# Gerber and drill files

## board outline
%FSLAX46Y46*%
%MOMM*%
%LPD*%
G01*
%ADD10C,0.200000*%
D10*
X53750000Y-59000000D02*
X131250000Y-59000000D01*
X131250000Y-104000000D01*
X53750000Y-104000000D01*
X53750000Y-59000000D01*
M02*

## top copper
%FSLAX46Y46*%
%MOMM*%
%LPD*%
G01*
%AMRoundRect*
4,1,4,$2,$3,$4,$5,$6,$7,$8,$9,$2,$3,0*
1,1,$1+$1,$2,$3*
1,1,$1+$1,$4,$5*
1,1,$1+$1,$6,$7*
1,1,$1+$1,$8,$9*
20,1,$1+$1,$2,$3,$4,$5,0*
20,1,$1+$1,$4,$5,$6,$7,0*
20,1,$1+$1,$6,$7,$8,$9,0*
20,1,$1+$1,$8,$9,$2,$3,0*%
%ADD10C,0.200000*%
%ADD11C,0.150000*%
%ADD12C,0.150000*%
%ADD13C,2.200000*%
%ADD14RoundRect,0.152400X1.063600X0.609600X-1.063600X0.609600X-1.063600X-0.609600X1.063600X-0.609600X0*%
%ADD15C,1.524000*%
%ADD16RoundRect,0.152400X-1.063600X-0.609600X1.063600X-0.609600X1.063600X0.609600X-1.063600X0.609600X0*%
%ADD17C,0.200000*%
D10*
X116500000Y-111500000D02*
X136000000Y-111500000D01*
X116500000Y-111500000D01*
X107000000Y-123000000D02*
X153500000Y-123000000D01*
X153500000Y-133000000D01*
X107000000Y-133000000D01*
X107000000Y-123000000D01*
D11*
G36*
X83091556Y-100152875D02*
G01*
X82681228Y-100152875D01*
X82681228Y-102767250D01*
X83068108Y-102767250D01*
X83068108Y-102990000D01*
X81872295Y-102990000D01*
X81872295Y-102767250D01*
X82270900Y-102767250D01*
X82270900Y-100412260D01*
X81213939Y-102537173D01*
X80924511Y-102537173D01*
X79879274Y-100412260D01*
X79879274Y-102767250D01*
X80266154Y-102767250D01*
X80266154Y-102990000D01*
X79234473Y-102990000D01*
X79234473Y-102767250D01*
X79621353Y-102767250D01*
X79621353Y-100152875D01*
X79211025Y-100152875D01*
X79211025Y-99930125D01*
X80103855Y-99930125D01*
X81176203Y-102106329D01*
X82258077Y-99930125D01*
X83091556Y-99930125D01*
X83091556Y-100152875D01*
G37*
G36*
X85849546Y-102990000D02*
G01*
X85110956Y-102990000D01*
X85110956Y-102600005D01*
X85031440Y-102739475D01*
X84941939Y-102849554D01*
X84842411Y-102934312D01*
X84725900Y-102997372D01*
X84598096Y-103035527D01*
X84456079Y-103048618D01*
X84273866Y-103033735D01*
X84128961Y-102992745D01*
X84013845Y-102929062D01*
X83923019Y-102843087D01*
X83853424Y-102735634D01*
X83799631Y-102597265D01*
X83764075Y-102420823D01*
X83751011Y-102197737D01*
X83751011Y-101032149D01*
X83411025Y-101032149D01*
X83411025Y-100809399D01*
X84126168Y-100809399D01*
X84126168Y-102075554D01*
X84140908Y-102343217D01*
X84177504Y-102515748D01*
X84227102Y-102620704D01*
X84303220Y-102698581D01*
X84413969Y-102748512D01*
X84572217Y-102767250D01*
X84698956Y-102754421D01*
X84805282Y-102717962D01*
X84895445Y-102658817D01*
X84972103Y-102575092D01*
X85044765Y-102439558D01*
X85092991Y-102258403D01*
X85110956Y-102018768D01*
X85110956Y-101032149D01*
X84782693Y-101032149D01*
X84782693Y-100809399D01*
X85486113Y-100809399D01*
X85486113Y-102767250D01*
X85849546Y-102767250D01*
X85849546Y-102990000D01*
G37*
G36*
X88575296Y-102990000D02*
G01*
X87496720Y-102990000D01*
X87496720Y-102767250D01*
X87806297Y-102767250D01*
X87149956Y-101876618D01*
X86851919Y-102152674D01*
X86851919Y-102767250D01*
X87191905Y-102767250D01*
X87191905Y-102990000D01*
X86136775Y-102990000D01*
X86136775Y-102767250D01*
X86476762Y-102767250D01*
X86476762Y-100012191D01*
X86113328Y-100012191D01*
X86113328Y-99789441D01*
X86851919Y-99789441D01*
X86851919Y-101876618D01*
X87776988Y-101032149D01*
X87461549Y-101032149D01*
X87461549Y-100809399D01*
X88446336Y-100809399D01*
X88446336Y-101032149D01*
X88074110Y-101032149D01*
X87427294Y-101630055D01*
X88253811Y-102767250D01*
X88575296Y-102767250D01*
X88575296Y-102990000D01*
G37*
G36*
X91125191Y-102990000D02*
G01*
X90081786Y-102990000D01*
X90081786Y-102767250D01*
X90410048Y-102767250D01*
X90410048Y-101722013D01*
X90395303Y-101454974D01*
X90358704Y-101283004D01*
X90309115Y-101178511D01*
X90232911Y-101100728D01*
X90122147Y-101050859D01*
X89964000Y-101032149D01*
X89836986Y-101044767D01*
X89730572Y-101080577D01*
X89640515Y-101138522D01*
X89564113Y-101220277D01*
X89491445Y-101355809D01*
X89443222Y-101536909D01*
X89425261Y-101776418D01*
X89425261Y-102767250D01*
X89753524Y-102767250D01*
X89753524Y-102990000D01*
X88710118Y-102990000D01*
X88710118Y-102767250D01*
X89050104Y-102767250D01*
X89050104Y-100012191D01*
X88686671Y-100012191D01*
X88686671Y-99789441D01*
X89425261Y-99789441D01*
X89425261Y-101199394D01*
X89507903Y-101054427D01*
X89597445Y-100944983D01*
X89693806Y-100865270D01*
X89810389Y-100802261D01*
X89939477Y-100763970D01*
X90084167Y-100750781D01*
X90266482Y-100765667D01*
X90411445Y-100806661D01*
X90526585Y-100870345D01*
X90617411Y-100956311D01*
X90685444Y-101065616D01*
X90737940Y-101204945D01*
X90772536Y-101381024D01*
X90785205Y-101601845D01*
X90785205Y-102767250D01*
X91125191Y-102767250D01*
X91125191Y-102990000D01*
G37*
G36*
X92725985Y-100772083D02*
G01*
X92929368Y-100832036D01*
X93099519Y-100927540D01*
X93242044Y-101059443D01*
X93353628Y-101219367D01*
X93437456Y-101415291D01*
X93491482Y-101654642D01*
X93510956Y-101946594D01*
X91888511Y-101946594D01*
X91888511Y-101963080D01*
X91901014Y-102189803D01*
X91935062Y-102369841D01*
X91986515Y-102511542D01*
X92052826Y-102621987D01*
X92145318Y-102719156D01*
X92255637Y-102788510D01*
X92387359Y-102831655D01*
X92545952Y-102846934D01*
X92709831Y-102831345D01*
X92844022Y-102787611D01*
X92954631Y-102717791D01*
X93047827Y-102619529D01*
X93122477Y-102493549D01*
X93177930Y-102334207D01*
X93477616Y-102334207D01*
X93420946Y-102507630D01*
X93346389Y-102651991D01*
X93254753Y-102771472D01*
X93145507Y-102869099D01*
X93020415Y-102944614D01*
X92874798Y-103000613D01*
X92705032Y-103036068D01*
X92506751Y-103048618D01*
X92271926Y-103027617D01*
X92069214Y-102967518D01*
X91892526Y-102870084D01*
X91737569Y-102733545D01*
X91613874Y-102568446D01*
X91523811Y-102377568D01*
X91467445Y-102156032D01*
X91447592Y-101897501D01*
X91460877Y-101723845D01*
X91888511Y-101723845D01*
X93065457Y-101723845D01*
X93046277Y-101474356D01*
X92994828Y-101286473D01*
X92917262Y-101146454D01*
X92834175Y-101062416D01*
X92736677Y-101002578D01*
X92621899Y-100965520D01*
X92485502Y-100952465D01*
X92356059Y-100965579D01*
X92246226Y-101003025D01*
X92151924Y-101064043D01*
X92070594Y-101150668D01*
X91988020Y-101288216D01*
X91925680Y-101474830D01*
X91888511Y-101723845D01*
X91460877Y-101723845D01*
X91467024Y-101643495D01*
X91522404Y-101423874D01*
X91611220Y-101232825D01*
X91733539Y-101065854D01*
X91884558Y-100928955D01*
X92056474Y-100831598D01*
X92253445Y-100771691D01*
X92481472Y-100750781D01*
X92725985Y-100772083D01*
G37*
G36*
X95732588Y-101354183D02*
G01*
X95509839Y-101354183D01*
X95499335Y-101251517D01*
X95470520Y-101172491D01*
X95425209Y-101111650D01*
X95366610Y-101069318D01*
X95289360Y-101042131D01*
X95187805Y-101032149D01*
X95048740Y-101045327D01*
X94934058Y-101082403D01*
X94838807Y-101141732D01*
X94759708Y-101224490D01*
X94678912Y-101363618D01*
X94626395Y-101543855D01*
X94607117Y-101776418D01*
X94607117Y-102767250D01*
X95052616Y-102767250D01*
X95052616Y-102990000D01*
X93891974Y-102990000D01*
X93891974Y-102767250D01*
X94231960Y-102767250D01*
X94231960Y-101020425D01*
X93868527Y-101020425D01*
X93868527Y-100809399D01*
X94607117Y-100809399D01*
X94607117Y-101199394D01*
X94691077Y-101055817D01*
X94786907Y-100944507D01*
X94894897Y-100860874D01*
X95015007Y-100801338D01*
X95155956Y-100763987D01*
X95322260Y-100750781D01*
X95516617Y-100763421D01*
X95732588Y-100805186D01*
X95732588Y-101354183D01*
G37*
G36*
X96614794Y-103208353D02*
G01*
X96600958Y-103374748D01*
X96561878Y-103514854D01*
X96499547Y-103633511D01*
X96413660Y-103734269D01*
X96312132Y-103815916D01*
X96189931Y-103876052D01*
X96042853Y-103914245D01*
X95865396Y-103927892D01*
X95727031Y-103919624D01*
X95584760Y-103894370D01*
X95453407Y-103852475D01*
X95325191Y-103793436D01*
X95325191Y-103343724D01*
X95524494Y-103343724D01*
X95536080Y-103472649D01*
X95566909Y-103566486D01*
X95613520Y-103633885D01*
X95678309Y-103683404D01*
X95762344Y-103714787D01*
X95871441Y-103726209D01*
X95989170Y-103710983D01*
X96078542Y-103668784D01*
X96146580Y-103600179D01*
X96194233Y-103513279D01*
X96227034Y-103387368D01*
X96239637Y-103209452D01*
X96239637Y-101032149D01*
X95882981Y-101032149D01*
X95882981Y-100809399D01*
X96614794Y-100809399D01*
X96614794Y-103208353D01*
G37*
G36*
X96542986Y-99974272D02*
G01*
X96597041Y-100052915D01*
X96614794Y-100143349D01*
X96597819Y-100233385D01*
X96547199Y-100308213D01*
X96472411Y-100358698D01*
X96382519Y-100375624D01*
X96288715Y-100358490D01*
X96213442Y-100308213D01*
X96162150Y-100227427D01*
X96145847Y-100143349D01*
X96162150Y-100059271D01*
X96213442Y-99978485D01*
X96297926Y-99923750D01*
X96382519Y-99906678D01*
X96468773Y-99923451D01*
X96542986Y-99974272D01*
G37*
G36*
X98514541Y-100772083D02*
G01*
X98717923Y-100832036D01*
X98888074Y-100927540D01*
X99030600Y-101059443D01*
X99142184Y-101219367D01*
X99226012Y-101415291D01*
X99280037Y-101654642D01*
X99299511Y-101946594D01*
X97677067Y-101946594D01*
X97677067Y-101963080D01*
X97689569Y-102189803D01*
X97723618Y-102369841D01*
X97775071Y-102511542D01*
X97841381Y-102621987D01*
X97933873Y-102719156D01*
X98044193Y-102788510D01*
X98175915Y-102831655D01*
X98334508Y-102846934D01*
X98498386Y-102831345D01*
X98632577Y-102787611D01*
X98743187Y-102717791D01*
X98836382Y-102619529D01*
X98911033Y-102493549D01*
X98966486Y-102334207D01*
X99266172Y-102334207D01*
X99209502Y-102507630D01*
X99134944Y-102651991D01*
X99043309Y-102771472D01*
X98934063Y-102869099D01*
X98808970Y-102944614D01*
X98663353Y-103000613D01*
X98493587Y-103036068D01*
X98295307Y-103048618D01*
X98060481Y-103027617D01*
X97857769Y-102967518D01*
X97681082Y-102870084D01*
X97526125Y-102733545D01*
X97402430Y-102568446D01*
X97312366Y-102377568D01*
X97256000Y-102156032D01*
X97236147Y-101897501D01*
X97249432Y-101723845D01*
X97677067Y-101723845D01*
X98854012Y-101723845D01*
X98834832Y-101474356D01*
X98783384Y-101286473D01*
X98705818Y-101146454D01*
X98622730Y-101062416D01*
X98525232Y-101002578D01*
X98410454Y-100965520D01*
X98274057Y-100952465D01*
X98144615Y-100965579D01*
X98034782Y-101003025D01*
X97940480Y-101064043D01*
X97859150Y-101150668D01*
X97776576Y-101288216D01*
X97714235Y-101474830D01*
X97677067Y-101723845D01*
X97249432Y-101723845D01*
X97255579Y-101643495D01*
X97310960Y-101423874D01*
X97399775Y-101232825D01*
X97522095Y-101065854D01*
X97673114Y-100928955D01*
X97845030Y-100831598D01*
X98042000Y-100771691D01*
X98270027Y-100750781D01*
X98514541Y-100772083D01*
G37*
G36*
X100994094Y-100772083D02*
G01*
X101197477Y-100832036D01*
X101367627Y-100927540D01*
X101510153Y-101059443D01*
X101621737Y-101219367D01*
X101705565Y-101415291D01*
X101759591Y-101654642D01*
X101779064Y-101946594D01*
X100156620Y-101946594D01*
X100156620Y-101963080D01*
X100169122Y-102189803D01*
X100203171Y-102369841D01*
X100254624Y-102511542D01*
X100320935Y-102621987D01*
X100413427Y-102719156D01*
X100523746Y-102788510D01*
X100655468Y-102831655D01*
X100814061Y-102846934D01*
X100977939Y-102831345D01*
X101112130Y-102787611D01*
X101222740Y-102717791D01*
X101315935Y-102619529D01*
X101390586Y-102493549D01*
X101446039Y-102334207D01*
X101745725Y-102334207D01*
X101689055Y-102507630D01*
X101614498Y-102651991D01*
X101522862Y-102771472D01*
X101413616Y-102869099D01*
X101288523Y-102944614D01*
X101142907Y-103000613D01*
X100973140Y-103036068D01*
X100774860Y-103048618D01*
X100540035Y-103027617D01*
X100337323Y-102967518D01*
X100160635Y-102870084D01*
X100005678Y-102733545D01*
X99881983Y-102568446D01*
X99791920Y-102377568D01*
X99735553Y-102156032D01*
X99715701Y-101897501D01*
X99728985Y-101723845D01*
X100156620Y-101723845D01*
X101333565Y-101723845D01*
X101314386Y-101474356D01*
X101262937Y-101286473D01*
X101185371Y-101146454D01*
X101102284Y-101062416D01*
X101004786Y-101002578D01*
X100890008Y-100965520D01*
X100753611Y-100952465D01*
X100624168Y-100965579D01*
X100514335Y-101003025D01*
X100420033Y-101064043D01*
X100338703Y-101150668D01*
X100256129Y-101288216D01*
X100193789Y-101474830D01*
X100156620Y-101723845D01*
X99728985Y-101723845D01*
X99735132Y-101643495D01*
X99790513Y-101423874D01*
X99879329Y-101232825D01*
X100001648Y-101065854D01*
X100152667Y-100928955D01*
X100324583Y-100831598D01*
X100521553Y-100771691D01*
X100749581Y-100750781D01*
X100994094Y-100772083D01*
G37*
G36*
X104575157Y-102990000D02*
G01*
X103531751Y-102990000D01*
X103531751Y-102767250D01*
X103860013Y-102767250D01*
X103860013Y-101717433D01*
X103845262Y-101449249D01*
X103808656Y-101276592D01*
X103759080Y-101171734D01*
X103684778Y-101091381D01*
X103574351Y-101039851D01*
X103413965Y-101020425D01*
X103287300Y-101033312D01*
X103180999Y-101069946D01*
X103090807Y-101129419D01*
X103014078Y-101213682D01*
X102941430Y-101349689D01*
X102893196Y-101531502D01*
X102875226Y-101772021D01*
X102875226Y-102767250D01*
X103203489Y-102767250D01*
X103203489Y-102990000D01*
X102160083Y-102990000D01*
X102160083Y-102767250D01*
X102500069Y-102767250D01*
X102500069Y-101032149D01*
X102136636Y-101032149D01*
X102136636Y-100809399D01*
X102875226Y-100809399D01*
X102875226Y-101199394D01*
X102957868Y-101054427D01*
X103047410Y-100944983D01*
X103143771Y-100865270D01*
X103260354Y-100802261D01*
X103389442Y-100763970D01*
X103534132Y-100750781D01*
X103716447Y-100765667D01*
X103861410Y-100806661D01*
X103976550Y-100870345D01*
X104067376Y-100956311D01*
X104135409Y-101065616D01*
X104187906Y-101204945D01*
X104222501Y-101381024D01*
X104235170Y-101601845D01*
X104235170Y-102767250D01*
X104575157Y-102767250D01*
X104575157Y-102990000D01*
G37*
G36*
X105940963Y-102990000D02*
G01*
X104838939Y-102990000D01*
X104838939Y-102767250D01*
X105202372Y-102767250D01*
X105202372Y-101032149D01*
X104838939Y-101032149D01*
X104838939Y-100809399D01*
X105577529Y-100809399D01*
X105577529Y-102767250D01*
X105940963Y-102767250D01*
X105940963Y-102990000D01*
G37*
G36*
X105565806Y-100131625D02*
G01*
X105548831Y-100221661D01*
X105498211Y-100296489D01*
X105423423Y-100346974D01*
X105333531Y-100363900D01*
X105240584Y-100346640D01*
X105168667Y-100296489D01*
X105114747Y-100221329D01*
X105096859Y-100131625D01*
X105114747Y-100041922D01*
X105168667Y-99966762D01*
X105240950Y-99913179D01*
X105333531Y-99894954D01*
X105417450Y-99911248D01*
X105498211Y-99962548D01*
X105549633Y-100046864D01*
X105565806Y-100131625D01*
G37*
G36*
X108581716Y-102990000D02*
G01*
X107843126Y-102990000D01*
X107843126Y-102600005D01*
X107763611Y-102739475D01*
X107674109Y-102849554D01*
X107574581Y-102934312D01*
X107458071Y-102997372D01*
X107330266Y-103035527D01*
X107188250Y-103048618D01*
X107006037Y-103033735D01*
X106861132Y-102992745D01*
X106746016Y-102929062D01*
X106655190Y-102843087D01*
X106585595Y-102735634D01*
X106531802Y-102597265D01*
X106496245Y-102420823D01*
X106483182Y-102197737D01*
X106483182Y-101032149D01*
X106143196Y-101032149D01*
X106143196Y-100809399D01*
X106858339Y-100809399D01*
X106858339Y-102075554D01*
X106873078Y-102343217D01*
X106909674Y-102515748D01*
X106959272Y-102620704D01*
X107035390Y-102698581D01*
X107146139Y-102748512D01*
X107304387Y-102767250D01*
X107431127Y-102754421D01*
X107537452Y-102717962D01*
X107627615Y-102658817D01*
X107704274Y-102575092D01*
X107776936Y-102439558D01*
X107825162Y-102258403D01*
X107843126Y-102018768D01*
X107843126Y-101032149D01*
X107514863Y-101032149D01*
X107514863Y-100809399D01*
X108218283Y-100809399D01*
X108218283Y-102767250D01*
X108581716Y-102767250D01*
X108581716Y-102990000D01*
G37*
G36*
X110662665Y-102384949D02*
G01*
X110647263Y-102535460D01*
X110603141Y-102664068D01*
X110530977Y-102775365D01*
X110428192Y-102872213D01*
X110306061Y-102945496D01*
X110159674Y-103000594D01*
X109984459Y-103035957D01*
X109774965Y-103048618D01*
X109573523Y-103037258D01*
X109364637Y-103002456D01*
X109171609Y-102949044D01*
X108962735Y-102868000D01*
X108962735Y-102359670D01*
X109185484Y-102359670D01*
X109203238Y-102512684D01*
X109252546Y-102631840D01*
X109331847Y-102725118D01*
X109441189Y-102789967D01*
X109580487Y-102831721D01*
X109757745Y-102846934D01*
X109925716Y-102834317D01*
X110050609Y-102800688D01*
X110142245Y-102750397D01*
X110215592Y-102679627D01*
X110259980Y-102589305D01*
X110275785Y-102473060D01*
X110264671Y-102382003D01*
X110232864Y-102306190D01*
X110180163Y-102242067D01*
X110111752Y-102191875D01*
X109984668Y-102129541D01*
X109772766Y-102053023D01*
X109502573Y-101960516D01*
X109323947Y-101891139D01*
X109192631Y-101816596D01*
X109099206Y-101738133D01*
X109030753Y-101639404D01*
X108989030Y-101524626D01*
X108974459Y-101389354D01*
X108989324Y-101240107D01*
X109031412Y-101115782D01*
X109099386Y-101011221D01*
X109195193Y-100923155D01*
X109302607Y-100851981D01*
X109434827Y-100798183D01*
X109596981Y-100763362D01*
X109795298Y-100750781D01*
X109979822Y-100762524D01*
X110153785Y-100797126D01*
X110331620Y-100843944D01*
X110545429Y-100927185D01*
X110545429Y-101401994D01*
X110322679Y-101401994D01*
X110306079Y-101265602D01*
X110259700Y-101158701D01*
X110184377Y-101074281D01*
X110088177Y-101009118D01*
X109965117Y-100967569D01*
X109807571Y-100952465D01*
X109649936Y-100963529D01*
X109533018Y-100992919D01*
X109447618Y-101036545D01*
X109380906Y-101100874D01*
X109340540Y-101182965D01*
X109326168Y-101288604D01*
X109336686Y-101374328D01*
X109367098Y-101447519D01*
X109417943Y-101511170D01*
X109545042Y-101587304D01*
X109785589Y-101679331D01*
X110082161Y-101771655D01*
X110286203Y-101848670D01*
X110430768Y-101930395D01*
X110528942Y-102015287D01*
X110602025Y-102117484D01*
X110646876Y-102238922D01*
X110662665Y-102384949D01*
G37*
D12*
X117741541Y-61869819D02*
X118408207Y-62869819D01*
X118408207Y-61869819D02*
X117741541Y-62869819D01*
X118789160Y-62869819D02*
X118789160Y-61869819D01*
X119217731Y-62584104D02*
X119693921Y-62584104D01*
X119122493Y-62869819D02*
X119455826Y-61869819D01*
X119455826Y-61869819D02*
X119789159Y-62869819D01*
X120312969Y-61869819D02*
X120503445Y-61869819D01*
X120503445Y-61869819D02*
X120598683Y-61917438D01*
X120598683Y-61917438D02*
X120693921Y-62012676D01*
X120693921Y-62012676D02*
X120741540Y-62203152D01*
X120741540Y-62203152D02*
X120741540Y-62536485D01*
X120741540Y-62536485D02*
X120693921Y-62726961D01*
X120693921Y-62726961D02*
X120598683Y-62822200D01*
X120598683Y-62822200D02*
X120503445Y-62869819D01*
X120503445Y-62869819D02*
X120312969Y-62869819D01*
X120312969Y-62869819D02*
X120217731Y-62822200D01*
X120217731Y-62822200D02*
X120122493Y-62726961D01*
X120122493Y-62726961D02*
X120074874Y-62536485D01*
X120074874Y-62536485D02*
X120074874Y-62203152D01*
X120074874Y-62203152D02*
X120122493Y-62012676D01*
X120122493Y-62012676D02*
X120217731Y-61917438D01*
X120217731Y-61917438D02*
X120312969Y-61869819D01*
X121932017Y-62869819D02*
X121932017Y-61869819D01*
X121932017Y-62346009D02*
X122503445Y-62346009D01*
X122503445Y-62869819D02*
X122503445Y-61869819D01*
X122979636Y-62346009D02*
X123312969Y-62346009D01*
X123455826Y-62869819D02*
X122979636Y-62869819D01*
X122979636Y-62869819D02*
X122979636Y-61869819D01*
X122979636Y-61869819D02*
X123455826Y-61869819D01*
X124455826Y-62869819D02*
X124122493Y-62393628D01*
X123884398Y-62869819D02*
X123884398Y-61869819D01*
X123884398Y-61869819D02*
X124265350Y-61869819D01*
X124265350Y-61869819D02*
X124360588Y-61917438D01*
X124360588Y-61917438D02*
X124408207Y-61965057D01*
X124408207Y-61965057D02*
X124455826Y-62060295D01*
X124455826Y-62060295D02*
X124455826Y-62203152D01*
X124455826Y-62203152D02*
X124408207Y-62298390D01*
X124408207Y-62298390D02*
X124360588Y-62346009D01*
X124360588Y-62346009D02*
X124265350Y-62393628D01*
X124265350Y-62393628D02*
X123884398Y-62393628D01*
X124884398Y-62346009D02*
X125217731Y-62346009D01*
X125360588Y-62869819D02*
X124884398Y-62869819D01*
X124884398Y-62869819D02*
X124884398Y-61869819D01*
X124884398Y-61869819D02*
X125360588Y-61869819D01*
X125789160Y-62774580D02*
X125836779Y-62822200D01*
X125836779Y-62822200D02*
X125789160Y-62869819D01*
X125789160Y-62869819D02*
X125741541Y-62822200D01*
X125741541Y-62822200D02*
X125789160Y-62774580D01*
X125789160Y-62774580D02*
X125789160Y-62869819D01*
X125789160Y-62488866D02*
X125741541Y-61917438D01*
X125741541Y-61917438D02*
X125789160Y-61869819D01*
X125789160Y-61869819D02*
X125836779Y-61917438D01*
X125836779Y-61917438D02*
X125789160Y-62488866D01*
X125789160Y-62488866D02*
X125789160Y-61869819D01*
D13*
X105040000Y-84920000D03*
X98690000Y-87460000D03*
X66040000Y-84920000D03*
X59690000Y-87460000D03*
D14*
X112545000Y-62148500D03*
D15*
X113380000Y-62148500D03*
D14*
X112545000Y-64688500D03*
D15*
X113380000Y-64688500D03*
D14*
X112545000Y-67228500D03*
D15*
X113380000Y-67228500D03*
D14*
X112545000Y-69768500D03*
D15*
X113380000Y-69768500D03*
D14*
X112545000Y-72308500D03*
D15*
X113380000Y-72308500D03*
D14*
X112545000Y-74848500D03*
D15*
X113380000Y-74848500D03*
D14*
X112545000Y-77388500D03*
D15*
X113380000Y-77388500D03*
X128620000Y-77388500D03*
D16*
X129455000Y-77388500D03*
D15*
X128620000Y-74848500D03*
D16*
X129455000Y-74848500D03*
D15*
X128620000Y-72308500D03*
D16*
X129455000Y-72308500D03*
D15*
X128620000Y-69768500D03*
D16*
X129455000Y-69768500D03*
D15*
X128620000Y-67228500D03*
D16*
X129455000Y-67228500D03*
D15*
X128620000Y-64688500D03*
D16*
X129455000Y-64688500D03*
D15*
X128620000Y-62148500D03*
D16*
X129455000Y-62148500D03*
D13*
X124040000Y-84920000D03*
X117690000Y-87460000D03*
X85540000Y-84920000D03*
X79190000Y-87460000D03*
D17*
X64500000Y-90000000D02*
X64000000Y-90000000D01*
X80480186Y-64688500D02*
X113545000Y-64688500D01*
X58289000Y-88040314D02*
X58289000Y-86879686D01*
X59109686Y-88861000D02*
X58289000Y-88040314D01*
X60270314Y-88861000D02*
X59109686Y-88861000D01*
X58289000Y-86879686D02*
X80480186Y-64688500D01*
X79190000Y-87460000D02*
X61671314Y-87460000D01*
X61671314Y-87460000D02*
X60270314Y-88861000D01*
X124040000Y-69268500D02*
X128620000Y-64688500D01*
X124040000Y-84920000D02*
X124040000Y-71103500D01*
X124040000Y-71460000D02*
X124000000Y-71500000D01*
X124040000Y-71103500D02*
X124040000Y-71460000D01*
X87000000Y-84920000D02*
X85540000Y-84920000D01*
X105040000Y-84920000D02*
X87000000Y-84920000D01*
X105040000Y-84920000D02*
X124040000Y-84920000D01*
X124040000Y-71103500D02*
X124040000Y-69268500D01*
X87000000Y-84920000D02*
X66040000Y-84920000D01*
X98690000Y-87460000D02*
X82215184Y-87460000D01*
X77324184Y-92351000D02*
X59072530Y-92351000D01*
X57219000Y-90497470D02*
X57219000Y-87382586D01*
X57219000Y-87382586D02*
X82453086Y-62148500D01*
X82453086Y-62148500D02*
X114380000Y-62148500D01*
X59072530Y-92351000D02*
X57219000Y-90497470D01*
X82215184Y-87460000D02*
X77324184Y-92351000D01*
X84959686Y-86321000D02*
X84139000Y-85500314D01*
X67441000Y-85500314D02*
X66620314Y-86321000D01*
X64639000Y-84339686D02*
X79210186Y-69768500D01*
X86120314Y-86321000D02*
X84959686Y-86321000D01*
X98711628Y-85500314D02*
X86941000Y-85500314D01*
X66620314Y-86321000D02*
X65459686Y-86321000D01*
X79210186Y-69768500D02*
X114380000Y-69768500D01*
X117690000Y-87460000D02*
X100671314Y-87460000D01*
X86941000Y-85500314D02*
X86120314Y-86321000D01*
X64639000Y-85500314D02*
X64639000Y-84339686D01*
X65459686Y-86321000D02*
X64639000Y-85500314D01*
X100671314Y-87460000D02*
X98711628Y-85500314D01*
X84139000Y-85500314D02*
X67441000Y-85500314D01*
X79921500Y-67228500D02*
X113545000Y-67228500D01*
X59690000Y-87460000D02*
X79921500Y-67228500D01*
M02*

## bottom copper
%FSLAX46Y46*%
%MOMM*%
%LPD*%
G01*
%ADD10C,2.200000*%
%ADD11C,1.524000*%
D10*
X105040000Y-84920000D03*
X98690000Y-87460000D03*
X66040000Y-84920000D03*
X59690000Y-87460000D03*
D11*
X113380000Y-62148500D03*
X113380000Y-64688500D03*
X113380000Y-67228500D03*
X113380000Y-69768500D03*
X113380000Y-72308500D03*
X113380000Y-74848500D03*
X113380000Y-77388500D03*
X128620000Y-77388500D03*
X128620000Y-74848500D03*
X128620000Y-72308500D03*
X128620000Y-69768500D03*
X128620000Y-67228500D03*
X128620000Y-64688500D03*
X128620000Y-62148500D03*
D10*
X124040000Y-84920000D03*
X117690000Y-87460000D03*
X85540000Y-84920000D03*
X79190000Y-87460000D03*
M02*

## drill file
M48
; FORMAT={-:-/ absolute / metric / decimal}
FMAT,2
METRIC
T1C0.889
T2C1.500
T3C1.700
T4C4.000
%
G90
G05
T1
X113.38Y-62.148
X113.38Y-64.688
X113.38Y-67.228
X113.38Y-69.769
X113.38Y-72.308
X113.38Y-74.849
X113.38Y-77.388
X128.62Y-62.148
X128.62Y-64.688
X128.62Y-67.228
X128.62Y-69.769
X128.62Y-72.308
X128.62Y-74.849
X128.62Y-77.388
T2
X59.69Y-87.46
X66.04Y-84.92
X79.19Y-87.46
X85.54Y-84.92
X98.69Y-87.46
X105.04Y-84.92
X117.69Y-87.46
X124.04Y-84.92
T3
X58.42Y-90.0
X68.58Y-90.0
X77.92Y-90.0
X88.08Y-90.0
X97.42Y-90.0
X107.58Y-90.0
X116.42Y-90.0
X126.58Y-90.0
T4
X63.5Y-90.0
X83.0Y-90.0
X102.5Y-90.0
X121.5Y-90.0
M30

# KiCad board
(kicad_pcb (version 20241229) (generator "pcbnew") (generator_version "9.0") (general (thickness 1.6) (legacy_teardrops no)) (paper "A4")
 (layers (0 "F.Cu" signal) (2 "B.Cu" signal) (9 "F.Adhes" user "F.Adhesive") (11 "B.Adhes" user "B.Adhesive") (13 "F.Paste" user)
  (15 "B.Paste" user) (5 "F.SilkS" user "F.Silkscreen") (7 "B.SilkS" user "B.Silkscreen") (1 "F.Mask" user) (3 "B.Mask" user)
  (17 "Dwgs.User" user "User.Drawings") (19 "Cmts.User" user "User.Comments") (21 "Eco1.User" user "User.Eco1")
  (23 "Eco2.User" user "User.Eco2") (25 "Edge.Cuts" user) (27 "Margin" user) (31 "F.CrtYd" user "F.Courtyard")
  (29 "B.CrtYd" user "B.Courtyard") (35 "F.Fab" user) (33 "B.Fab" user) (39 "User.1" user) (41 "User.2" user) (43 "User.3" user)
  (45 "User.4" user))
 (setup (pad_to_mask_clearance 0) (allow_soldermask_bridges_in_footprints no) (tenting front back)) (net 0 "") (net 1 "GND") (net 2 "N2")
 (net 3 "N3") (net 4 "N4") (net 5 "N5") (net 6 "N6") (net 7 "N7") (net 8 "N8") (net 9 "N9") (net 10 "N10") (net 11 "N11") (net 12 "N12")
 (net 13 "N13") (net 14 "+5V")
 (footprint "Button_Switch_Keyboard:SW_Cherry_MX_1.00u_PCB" (layer "F.Cu") (at 105.04 84.92)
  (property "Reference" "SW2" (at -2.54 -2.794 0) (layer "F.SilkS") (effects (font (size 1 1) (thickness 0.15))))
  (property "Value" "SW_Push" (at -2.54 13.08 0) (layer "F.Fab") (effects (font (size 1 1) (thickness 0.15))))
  (pad "" np_thru_hole circle (at -7.62 5.08) (size 1.7 1.7) (drill 1.7) (layers "*.Cu" "*.Mask"))
  (pad "" np_thru_hole circle (at -2.54 5.08) (size 4 4) (drill 4) (layers "*.Cu" "*.Mask"))
  (pad "" np_thru_hole circle (at 2.54 5.08) (size 1.7 1.7) (drill 1.7) (layers "*.Cu" "*.Mask"))
  (pad "1" thru_hole circle (at 0 0) (size 2.2 2.2) (drill 1.5) (layers "*.Cu" "*.Mask") (remove_unused_layers no) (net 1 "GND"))
  (pad "2" thru_hole circle (at -6.35 2.54) (size 2.2 2.2) (drill 1.5) (layers "*.Cu" "*.Mask") (remove_unused_layers no) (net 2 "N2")))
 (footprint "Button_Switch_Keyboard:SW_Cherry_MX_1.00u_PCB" (layer "F.Cu") (at 66.04 84.92)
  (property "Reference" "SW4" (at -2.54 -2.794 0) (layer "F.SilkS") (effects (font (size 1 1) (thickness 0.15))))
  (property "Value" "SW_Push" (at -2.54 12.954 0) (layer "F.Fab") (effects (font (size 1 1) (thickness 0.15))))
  (pad "" np_thru_hole circle (at -7.62 5.08) (size 1.7 1.7) (drill 1.7) (layers "*.Cu" "*.Mask"))
  (pad "" np_thru_hole circle (at -2.54 5.08) (size 4 4) (drill 4) (layers "*.Cu" "*.Mask"))
  (pad "" np_thru_hole circle (at 2.54 5.08) (size 1.7 1.7) (drill 1.7) (layers "*.Cu" "*.Mask"))
  (pad "1" thru_hole circle (at 0 0) (size 2.2 2.2) (drill 1.5) (layers "*.Cu" "*.Mask") (remove_unused_layers no) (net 1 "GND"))
  (pad "2" thru_hole circle (at -6.35 2.54) (size 2.2 2.2) (drill 1.5) (layers "*.Cu" "*.Mask") (remove_unused_layers no) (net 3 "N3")))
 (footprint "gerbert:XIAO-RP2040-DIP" (layer "F.Cu") (at 121 69.7685)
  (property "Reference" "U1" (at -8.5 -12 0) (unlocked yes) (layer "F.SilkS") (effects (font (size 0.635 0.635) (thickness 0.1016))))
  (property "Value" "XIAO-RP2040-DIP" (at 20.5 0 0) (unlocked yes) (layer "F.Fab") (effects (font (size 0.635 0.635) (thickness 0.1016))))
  (pad "1" smd roundrect (at -8.455 -7.62 180) (size 2.432 1.524) (layers "F.Cu" "F.Mask") (roundrect_rratio 0.1) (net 2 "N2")
   (thermal_bridge_angle 45))
  (pad "1" thru_hole circle (at -7.62 -7.62 180) (size 1.524 1.524) (drill 0.889) (layers "*.Cu" "*.Mask") (remove_unused_layers no)
   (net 2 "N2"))
  (pad "2" smd roundrect (at -8.455 -5.08 180) (size 2.432 1.524) (layers "F.Cu" "F.Mask") (roundrect_rratio 0.1) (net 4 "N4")
   (thermal_bridge_angle 45))
  (pad "2" thru_hole circle (at -7.62 -5.08 180) (size 1.524 1.524) (drill 0.889) (layers "*.Cu" "*.Mask") (remove_unused_layers no)
   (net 4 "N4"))
  (pad "3" smd roundrect (at -8.455 -2.54 180) (size 2.432 1.524) (layers "F.Cu" "F.Mask") (roundrect_rratio 0.1) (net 3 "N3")
   (thermal_bridge_angle 45))
  (pad "3" thru_hole circle (at -7.62 -2.54 180) (size 1.524 1.524) (drill 0.889) (layers "*.Cu" "*.Mask") (remove_unused_layers no)
   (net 3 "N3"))
  (pad "4" smd roundrect (at -8.455 0 180) (size 2.432 1.524) (layers "F.Cu" "F.Mask") (roundrect_rratio 0.1) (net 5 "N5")
   (thermal_bridge_angle 45))
  (pad "4" thru_hole circle (at -7.62 0 180) (size 1.524 1.524) (drill 0.889) (layers "*.Cu" "*.Mask") (remove_unused_layers no)
   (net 5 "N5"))
  (pad "5" smd roundrect (at -8.455 2.54 180) (size 2.432 1.524) (layers "F.Cu" "F.Mask") (roundrect_rratio 0.1) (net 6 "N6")
   (thermal_bridge_angle 45))
  (pad "5" thru_hole circle (at -7.62 2.54 180) (size 1.524 1.524) (drill 0.889) (layers "*.Cu" "*.Mask") (remove_unused_layers no)
   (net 6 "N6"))
  (pad "6" smd roundrect (at -8.455 5.08 180) (size 2.432 1.524) (layers "F.Cu" "F.Mask") (roundrect_rratio 0.1) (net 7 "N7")
   (thermal_bridge_angle 45))
  (pad "6" thru_hole circle (at -7.62 5.08 180) (size 1.524 1.524) (drill 0.889) (layers "*.Cu" "*.Mask") (remove_unused_layers no)
   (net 7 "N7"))
  (pad "7" smd roundrect (at -8.455 7.62 180) (size 2.432 1.524) (layers "F.Cu" "F.Mask") (roundrect_rratio 0.1) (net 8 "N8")
   (thermal_bridge_angle 45))
  (pad "7" thru_hole circle (at -7.62 7.62 180) (size 1.524 1.524) (drill 0.889) (layers "*.Cu" "*.Mask") (remove_unused_layers no)
   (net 8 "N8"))
  (pad "8" thru_hole circle (at 7.62 7.62) (size 1.524 1.524) (drill 0.889) (layers "*.Cu" "*.Mask") (remove_unused_layers no) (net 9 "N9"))
  (pad "8" smd roundrect (at 8.455 7.62) (size 2.432 1.524) (layers "F.Cu" "F.Mask") (roundrect_rratio 0.1) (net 9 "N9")
   (thermal_bridge_angle 45))
  (pad "9" thru_hole circle (at 7.62 5.08) (size 1.524 1.524) (drill 0.889) (layers "*.Cu" "*.Mask") (remove_unused_layers no)
   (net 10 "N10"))
  (pad "9" smd roundrect (at 8.455 5.08) (size 2.432 1.524) (layers "F.Cu" "F.Mask") (roundrect_rratio 0.1) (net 10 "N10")
   (thermal_bridge_angle 45))
  (pad "10" thru_hole circle (at 7.62 2.54) (size 1.524 1.524) (drill 0.889) (layers "*.Cu" "*.Mask") (remove_unused_layers no)
   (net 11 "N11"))
  (pad "10" smd roundrect (at 8.455 2.54) (size 2.432 1.524) (layers "F.Cu" "F.Mask") (roundrect_rratio 0.1) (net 11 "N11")
   (thermal_bridge_angle 45))
  (pad "11" thru_hole circle (at 7.62 0) (size 1.524 1.524) (drill 0.889) (layers "*.Cu" "*.Mask") (remove_unused_layers no) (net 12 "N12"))
  (pad "11" smd roundrect (at 8.455 0) (size 2.432 1.524) (layers "F.Cu" "F.Mask") (roundrect_rratio 0.1) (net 12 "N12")
   (thermal_bridge_angle 45))
  (pad "12" thru_hole circle (at 7.62 -2.54) (size 1.524 1.524) (drill 0.889) (layers "*.Cu" "*.Mask") (remove_unused_layers no)
   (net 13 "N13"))
  (pad "12" smd roundrect (at 8.455 -2.54) (size 2.432 1.524) (layers "F.Cu" "F.Mask") (roundrect_rratio 0.1) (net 13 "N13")
   (thermal_bridge_angle 45))
  (pad "13" thru_hole circle (at 7.62 -5.08) (size 1.524 1.524) (drill 0.889) (layers "*.Cu" "*.Mask") (remove_unused_layers no)
   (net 1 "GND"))
  (pad "13" smd roundrect (at 8.455 -5.08) (size 2.432 1.524) (layers "F.Cu" "F.Mask") (roundrect_rratio 0.1) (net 1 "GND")
   (thermal_bridge_angle 45))
  (pad "14" thru_hole circle (at 7.62 -7.62) (size 1.524 1.524) (drill 0.889) (layers "*.Cu" "*.Mask") (remove_unused_layers no)
   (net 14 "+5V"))
  (pad "14" smd roundrect (at 8.455 -7.62) (size 2.432 1.524) (layers "F.Cu" "F.Mask") (roundrect_rratio 0.1) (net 14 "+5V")
   (thermal_bridge_angle 45)))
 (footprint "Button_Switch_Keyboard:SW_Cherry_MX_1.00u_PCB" (layer "F.Cu") (at 124.04 84.92)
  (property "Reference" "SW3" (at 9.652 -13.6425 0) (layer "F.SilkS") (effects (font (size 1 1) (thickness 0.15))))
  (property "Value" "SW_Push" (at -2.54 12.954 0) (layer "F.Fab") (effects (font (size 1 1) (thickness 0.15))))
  (pad "" np_thru_hole circle (at -7.62 5.08) (size 1.7 1.7) (drill 1.7) (layers "*.Cu" "*.Mask"))
  (pad "" np_thru_hole circle (at -2.54 5.08) (size 4 4) (drill 4) (layers "*.Cu" "*.Mask"))
  (pad "" np_thru_hole circle (at 2.54 5.08) (size 1.7 1.7) (drill 1.7) (layers "*.Cu" "*.Mask"))
  (pad "1" thru_hole circle (at 0 0) (size 2.2 2.2) (drill 1.5) (layers "*.Cu" "*.Mask") (remove_unused_layers no) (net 1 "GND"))
  (pad "2" thru_hole circle (at -6.35 2.54) (size 2.2 2.2) (drill 1.5) (layers "*.Cu" "*.Mask") (remove_unused_layers no) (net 5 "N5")))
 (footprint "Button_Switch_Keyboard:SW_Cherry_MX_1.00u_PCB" (layer "F.Cu") (at 85.54 84.92)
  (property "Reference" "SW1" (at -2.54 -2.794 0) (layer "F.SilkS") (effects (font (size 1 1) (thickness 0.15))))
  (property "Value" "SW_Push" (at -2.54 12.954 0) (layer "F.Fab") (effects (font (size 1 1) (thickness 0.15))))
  (pad "" np_thru_hole circle (at -7.62 5.08) (size 1.7 1.7) (drill 1.7) (layers "*.Cu" "*.Mask"))
  (pad "" np_thru_hole circle (at -2.54 5.08) (size 4 4) (drill 4) (layers "*.Cu" "*.Mask"))
  (pad "" np_thru_hole circle (at 2.54 5.08) (size 1.7 1.7) (drill 1.7) (layers "*.Cu" "*.Mask"))
  (pad "1" thru_hole circle (at 0 0) (size 2.2 2.2) (drill 1.5) (layers "*.Cu" "*.Mask") (remove_unused_layers no) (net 1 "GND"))
  (pad "2" thru_hole circle (at -6.35 2.54) (size 2.2 2.2) (drill 1.5) (layers "*.Cu" "*.Mask") (remove_unused_layers no) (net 4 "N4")))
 (gr_rect (start 116.5 111.5) (end 136 111.5) (stroke (width 0.2) (type default)) (fill no) (layer "F.Cu"))
 (gr_rect (start 107 123) (end 153.5 133) (stroke (width 0.2) (type default)) (fill no) (layer "F.Cu"))
 (gr_rect (start 53.75 59) (end 131.25 104) (stroke (width 0.2) (type solid)) (fill no) (layer "Edge.Cuts"))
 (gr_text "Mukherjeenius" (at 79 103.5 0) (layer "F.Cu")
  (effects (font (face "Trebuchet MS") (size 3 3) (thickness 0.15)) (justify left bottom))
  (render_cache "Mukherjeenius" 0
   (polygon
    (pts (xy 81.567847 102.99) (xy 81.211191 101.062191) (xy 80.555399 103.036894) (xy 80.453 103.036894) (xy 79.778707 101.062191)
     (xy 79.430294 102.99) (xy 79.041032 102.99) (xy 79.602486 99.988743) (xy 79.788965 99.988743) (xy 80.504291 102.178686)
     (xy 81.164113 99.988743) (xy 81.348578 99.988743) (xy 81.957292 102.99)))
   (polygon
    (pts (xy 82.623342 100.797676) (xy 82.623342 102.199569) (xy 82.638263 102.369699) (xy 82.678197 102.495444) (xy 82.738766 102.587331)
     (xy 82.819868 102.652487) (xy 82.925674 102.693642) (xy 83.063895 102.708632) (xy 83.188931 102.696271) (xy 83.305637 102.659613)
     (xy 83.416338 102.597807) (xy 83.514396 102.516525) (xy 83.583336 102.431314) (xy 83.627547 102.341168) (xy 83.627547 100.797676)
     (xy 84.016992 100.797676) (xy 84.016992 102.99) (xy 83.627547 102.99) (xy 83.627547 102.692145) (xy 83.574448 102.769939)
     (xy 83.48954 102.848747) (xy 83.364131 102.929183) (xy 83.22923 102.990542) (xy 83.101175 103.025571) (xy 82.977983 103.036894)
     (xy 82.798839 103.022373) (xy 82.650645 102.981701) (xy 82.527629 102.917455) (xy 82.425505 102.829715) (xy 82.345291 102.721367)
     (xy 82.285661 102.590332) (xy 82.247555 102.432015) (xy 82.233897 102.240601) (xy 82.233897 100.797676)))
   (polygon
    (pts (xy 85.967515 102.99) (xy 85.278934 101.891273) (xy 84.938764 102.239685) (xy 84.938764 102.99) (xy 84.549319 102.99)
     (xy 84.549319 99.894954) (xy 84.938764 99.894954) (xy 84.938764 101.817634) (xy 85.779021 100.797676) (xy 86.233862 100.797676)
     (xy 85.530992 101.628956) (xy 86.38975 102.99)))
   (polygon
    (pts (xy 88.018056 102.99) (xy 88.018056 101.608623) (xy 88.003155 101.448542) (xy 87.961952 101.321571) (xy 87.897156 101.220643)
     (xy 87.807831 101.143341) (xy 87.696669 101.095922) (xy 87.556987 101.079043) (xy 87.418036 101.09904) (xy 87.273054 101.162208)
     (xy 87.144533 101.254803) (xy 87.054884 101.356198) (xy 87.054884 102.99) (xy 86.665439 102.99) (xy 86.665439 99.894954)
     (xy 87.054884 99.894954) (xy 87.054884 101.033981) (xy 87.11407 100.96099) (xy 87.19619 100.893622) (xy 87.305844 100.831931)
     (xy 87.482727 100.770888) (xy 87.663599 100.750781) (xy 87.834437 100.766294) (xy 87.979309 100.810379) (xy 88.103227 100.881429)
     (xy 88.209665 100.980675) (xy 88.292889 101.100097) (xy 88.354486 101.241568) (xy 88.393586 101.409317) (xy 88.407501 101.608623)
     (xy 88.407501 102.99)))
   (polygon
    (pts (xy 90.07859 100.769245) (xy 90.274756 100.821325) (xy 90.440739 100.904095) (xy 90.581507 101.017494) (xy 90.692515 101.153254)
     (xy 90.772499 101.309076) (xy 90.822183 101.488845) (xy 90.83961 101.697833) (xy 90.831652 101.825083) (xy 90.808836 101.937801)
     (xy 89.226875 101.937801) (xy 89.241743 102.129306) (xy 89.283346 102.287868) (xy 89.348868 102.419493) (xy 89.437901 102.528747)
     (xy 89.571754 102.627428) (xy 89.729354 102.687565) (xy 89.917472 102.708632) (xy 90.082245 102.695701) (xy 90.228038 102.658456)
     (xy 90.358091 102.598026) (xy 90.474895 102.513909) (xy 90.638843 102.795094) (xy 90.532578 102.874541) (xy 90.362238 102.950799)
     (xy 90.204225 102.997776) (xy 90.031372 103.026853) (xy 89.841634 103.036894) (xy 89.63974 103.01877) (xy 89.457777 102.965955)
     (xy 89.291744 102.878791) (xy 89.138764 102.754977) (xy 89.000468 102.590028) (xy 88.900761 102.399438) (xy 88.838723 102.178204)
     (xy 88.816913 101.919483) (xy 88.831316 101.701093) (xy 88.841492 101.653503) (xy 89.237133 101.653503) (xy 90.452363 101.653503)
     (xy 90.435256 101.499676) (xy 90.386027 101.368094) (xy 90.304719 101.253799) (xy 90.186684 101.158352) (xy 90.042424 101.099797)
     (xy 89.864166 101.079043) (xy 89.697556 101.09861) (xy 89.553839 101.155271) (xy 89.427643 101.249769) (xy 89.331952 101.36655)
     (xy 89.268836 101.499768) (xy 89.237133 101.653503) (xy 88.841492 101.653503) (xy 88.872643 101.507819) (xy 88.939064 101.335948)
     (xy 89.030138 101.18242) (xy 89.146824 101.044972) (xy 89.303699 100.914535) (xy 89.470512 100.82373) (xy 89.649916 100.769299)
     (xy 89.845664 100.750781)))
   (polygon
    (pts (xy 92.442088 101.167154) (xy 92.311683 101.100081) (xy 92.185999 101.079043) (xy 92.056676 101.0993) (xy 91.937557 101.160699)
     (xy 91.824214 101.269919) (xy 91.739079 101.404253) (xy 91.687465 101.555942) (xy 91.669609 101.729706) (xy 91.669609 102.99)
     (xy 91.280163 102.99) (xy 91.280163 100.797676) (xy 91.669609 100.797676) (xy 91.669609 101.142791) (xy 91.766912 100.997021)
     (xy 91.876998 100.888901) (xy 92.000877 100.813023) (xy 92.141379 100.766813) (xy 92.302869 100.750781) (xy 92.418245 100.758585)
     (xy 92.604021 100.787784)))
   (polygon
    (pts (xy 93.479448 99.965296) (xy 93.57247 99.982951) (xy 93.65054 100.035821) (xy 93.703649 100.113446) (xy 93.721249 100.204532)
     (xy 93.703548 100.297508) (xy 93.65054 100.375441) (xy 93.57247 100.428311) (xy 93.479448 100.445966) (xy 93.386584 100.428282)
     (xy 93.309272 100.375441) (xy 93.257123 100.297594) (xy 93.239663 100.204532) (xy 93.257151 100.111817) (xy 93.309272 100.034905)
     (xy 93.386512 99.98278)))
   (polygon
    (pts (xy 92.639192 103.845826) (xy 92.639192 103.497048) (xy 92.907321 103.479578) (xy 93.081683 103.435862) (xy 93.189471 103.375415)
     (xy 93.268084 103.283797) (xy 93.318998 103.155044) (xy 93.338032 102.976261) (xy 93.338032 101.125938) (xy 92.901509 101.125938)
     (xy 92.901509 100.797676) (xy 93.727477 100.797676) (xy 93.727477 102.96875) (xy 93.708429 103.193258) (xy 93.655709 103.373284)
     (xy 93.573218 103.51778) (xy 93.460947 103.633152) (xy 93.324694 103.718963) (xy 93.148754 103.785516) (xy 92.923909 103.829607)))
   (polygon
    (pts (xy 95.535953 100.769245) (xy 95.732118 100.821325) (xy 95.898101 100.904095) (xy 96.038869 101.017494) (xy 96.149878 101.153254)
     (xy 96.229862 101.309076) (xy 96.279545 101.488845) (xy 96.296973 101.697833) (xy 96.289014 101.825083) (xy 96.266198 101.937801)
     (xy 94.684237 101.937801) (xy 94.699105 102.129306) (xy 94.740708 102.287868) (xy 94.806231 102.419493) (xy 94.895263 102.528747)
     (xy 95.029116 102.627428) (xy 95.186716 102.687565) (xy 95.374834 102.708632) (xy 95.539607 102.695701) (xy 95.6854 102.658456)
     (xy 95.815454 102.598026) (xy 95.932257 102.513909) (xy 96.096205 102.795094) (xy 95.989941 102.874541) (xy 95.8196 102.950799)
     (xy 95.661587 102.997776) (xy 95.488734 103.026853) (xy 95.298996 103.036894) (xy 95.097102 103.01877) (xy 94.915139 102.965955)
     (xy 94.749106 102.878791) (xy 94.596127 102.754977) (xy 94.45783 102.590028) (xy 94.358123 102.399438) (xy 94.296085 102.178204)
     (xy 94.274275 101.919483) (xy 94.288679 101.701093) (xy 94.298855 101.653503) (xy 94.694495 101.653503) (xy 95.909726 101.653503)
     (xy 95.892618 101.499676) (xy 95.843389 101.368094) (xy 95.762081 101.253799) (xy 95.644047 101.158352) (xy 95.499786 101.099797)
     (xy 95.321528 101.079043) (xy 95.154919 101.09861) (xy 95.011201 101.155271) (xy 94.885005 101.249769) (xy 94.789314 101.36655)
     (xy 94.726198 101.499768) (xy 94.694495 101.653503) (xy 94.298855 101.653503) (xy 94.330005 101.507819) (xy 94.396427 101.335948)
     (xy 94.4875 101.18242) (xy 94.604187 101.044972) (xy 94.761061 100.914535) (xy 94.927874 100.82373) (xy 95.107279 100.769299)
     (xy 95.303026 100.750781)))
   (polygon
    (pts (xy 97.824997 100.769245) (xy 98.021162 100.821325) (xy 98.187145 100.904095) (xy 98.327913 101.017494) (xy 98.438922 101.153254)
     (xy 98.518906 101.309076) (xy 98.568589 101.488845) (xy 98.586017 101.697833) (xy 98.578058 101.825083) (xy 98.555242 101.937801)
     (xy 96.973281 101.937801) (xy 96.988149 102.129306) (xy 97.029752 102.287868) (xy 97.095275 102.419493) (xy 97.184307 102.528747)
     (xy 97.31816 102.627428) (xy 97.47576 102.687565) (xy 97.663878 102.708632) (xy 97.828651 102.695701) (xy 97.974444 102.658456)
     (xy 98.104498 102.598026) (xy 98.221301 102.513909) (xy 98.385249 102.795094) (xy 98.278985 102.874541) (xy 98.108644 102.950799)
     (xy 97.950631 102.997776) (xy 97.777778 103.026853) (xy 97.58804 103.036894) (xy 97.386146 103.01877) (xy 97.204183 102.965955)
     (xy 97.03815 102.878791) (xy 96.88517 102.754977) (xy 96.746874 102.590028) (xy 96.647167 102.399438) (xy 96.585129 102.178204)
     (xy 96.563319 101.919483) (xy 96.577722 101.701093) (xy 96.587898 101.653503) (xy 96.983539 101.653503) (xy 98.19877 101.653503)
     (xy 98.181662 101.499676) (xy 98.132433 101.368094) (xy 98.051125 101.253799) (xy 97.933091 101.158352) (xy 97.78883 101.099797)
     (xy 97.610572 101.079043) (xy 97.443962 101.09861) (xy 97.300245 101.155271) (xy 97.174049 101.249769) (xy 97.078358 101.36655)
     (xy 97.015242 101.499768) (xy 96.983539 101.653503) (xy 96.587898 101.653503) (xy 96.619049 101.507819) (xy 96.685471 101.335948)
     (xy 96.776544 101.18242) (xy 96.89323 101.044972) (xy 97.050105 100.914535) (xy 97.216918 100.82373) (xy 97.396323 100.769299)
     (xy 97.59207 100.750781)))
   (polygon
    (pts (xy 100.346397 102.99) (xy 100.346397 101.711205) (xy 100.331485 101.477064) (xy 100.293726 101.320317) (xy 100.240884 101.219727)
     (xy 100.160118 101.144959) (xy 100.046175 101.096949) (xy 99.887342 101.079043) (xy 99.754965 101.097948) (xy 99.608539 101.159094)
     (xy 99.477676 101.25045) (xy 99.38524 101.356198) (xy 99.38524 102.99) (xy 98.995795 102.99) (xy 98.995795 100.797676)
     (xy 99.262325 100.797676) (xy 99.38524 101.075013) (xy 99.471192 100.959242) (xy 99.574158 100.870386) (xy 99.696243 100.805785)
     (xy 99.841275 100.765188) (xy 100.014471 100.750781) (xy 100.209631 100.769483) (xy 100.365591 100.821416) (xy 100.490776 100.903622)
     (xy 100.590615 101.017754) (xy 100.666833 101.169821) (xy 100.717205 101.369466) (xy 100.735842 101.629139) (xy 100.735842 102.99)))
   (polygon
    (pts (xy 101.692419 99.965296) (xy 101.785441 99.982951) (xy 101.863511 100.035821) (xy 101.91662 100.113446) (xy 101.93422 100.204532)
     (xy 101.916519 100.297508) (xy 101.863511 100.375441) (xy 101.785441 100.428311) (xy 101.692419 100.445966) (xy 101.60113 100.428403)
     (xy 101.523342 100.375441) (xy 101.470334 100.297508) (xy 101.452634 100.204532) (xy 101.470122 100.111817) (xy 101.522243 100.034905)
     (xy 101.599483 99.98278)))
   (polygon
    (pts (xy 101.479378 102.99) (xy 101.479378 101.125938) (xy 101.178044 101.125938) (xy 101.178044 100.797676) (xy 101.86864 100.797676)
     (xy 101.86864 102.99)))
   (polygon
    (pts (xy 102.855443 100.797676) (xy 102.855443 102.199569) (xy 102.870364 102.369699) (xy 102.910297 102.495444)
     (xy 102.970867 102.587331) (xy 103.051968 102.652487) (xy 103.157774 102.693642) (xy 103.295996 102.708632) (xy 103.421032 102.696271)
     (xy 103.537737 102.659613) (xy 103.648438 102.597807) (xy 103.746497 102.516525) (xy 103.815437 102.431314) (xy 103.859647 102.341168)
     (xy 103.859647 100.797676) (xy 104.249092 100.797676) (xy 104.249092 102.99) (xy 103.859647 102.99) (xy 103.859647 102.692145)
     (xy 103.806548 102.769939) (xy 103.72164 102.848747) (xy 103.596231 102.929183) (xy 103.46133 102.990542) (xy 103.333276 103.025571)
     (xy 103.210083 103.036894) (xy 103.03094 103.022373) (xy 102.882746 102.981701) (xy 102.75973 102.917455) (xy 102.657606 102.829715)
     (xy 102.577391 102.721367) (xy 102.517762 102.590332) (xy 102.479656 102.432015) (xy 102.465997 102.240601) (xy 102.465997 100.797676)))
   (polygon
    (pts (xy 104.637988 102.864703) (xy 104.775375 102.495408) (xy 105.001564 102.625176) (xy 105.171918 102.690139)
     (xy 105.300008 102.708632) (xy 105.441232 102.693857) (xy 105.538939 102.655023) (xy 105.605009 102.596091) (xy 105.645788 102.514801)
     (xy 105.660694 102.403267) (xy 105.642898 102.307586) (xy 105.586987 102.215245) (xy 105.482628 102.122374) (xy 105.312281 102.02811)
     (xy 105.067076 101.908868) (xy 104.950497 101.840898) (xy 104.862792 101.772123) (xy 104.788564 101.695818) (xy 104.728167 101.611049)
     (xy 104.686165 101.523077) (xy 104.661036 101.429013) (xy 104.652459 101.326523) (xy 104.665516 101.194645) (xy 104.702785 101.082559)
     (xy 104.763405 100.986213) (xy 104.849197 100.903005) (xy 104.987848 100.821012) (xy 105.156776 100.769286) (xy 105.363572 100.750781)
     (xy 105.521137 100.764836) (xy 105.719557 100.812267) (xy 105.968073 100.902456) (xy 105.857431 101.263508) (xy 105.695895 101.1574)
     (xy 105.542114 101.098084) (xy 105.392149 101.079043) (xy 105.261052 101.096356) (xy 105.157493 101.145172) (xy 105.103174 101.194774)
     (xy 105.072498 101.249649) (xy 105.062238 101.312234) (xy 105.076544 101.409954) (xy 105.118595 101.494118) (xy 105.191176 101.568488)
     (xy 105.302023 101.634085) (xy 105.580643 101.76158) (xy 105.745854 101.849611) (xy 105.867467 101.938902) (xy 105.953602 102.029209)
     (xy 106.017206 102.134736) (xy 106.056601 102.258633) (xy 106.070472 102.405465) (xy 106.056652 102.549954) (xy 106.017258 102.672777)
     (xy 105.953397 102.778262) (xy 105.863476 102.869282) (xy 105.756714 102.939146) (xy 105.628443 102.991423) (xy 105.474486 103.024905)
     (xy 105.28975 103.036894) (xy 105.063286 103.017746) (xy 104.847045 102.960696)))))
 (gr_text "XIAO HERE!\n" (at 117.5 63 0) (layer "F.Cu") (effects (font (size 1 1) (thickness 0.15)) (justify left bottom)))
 (segment (start 64.5 90) (end 64 90) (width 0.2) (layer "F.Cu") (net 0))
 (segment (start 80.480186 64.6885) (end 113.545 64.6885) (width 0.2) (layer "F.Cu") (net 4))
 (segment (start 58.289 88.040314) (end 58.289 86.879686) (width 0.2) (layer "F.Cu") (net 4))
 (segment (start 59.109686 88.861) (end 58.289 88.040314) (width 0.2) (layer "F.Cu") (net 4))
 (segment (start 60.270314 88.861) (end 59.109686 88.861) (width 0.2) (layer "F.Cu") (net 4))
 (segment (start 58.289 86.879686) (end 80.480186 64.6885) (width 0.2) (layer "F.Cu") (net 4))
 (segment (start 79.19 87.46) (end 61.671314 87.46) (width 0.2) (layer "F.Cu") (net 4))
 (segment (start 61.671314 87.46) (end 60.270314 88.861) (width 0.2) (layer "F.Cu") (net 4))
 (segment (start 124.04 69.2685) (end 128.62 64.6885) (width 0.2) (layer "F.Cu") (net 1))
 (segment (start 124.04 84.92) (end 124.04 71.1035) (width 0.2) (layer "F.Cu") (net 1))
 (segment (start 124.04 71.46) (end 124 71.5) (width 0.2) (layer "F.Cu") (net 1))
 (segment (start 124.04 71.1035) (end 124.04 71.46) (width 0.2) (layer "F.Cu") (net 1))
 (segment (start 87 84.92) (end 85.54 84.92) (width 0.2) (layer "F.Cu") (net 1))
 (segment (start 105.04 84.92) (end 87 84.92) (width 0.2) (layer "F.Cu") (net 1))
 (segment (start 105.04 84.92) (end 124.04 84.92) (width 0.2) (layer "F.Cu") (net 1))
 (segment (start 124.04 71.1035) (end 124.04 69.2685) (width 0.2) (layer "F.Cu") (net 1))
 (segment (start 87 84.92) (end 66.04 84.92) (width 0.2) (layer "F.Cu") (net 1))
 (segment (start 98.69 87.46) (end 82.215184 87.46) (width 0.2) (layer "F.Cu") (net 2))
 (segment (start 77.324184 92.351) (end 59.07253 92.351) (width 0.2) (layer "F.Cu") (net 2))
 (segment (start 57.219 90.49747) (end 57.219 87.382586) (width 0.2) (layer "F.Cu") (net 2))
 (segment (start 57.219 87.382586) (end 82.453086 62.1485) (width 0.2) (layer "F.Cu") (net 2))
 (segment (start 82.453086 62.1485) (end 114.38 62.1485) (width 0.2) (layer "F.Cu") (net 2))
 (segment (start 59.07253 92.351) (end 57.219 90.49747) (width 0.2) (layer "F.Cu") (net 2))
 (segment (start 82.215184 87.46) (end 77.324184 92.351) (width 0.2) (layer "F.Cu") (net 2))
 (segment (start 84.959686 86.321) (end 84.139 85.500314) (width 0.2) (layer "F.Cu") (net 5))
 (segment (start 67.441 85.500314) (end 66.620314 86.321) (width 0.2) (layer "F.Cu") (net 5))
 (segment (start 64.639 84.339686) (end 79.210186 69.7685) (width 0.2) (layer "F.Cu") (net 5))
 (segment (start 86.120314 86.321) (end 84.959686 86.321) (width 0.2) (layer "F.Cu") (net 5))
 (segment (start 98.711628 85.500314) (end 86.941 85.500314) (width 0.2) (layer "F.Cu") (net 5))
 (segment (start 66.620314 86.321) (end 65.459686 86.321) (width 0.2) (layer "F.Cu") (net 5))
 (segment (start 79.210186 69.7685) (end 114.38 69.7685) (width 0.2) (layer "F.Cu") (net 5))
 (segment (start 117.69 87.46) (end 100.671314 87.46) (width 0.2) (layer "F.Cu") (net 5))
 (segment (start 86.941 85.500314) (end 86.120314 86.321) (width 0.2) (layer "F.Cu") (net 5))
 (segment (start 64.639 85.500314) (end 64.639 84.339686) (width 0.2) (layer "F.Cu") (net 5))
 (segment (start 65.459686 86.321) (end 64.639 85.500314) (width 0.2) (layer "F.Cu") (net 5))
 (segment (start 100.671314 87.46) (end 98.711628 85.500314) (width 0.2) (layer "F.Cu") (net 5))
 (segment (start 84.139 85.500314) (end 67.441 85.500314) (width 0.2) (layer "F.Cu") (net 5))
 (segment (start 79.9215 67.2285) (end 113.545 67.2285) (width 0.2) (layer "F.Cu") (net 3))
 (segment (start 59.69 87.46) (end 79.9215 67.2285) (width 0.2) (layer "F.Cu") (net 3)))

